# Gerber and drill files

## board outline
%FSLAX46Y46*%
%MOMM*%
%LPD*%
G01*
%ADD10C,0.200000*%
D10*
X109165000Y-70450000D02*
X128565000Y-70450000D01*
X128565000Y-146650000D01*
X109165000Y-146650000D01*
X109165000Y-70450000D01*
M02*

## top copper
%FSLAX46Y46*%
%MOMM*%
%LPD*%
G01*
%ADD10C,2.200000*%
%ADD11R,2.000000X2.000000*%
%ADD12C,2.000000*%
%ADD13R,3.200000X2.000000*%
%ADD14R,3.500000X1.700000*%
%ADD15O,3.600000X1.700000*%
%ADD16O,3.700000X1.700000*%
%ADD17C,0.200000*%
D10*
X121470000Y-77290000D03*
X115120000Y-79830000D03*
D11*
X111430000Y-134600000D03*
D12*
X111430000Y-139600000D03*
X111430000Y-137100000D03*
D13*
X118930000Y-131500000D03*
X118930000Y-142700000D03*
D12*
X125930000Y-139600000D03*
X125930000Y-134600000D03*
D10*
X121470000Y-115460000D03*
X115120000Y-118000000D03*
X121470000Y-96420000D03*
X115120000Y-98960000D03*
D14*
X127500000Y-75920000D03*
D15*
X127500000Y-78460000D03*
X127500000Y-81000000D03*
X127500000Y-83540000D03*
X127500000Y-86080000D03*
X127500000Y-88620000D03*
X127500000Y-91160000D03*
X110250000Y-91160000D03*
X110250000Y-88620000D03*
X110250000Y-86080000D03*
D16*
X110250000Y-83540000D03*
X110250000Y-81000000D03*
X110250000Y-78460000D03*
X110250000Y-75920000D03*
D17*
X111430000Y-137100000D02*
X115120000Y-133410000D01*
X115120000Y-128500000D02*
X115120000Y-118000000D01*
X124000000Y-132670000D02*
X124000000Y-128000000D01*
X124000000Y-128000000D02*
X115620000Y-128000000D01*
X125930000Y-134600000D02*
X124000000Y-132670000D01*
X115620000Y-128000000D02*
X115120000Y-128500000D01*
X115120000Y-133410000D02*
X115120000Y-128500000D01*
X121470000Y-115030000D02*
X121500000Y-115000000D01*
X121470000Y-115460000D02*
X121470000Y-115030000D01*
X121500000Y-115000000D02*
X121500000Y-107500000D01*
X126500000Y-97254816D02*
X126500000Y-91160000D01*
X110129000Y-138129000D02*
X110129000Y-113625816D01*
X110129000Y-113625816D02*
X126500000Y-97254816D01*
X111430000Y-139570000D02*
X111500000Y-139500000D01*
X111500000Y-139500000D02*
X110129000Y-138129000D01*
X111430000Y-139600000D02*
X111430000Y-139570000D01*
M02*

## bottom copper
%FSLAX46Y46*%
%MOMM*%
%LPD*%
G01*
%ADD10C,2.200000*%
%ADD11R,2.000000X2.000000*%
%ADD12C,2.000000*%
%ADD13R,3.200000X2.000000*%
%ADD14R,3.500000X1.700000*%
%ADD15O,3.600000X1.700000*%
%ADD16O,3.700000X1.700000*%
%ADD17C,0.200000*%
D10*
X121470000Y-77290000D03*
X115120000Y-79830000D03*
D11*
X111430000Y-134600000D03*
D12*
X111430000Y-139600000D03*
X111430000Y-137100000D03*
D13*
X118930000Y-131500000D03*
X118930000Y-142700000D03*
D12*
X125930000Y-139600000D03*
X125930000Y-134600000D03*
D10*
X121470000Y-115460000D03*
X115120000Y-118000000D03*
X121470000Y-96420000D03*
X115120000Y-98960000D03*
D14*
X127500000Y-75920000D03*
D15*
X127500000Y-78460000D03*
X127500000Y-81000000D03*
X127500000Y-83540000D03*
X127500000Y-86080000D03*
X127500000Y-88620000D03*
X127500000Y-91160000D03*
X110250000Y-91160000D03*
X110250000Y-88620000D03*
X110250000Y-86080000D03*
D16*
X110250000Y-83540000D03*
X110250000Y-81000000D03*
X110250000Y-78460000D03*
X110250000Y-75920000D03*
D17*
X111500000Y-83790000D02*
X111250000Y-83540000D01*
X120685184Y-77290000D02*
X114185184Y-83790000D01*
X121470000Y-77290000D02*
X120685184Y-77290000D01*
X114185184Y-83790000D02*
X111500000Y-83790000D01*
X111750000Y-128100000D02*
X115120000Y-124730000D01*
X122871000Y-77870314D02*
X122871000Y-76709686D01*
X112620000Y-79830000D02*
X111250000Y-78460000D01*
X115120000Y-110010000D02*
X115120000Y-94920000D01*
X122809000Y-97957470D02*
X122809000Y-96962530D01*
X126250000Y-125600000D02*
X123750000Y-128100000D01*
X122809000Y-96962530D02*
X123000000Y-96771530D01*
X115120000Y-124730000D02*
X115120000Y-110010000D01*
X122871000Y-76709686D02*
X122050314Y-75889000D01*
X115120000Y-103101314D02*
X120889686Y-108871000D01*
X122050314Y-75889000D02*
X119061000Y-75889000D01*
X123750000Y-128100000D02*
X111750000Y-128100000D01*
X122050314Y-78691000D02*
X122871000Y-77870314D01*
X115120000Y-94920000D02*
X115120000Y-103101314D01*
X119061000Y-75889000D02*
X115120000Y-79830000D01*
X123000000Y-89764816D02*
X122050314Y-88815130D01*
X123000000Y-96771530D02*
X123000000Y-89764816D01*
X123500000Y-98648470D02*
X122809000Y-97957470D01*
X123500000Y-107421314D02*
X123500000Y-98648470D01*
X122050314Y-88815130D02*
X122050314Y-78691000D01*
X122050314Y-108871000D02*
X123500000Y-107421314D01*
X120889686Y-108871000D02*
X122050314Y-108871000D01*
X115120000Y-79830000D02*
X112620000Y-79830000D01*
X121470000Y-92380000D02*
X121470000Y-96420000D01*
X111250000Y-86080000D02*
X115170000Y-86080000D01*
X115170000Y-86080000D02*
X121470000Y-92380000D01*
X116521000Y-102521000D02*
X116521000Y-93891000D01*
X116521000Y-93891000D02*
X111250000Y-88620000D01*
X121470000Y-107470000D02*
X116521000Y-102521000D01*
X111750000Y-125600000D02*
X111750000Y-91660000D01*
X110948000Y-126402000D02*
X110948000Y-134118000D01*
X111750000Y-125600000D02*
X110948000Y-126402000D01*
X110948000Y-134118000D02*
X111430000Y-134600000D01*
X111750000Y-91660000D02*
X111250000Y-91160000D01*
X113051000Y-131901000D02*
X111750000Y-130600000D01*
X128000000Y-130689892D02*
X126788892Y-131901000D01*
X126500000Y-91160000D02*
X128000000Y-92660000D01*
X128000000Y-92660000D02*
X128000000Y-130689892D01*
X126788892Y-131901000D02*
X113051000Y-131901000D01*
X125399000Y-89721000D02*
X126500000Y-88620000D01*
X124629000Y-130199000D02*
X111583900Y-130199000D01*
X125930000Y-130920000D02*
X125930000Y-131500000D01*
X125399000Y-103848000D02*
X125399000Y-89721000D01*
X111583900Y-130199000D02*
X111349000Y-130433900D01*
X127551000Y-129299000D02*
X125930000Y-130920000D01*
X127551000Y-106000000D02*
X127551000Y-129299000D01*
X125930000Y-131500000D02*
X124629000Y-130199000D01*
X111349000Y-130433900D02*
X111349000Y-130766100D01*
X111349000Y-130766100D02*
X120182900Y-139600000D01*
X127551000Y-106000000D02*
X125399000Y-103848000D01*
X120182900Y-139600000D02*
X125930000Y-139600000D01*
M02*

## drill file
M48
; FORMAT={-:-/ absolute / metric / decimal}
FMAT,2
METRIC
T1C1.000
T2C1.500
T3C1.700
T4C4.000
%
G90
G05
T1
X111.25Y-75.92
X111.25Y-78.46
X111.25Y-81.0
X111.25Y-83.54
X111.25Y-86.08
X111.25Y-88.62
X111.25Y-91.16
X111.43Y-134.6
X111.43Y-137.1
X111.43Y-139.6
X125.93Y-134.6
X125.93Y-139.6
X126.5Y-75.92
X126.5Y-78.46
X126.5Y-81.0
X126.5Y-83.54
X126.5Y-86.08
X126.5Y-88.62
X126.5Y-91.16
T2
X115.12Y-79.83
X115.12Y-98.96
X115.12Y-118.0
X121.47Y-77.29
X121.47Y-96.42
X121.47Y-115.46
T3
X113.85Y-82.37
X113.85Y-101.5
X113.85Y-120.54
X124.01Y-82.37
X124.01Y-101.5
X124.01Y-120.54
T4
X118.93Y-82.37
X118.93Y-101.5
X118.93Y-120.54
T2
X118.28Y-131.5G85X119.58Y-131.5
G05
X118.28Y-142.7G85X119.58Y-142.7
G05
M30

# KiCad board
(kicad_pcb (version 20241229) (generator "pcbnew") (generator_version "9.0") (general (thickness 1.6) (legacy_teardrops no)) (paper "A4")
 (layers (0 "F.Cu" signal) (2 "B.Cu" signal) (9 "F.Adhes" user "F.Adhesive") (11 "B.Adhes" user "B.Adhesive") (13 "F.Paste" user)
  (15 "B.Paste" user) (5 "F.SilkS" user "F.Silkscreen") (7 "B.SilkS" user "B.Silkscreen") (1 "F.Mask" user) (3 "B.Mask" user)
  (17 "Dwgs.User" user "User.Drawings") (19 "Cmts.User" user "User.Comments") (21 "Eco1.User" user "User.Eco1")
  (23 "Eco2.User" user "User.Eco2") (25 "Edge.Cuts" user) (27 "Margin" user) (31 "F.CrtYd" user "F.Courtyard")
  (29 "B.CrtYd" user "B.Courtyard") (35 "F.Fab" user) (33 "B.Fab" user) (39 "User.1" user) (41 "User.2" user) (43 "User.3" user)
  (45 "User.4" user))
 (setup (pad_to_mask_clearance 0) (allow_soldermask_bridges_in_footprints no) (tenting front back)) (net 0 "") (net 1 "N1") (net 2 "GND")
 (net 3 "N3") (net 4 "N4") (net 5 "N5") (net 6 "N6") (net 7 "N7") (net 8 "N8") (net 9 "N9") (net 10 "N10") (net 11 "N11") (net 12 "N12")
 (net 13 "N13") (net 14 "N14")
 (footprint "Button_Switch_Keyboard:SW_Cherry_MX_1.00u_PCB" (layer "F.Cu") (at 121.47 77.29)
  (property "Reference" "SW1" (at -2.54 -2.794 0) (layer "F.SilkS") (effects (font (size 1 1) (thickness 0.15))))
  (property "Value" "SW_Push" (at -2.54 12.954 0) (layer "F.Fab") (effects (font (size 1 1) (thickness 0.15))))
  (pad "" np_thru_hole circle (at -7.62 5.08) (size 1.7 1.7) (drill 1.7) (layers "*.Cu" "*.Mask"))
  (pad "" np_thru_hole circle (at -2.54 5.08) (size 4 4) (drill 4) (layers "*.Cu" "*.Mask"))
  (pad "" np_thru_hole circle (at 2.54 5.08) (size 1.7 1.7) (drill 1.7) (layers "*.Cu" "*.Mask"))
  (pad "1" thru_hole circle (at 0 0) (size 2.2 2.2) (drill 1.5) (layers "*.Cu" "*.Mask") (remove_unused_layers no) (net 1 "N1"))
  (pad "2" thru_hole circle (at -6.35 2.54) (size 2.2 2.2) (drill 1.5) (layers "*.Cu" "*.Mask") (remove_unused_layers no) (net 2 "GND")))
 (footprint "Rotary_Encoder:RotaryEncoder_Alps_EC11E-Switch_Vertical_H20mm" (layer "F.Cu") (at 111.43 134.6)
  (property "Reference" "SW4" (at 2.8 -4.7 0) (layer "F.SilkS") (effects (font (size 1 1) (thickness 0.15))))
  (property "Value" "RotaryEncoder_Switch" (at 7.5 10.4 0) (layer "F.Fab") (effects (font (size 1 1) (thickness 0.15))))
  (pad "A" thru_hole rect (at 0 0) (size 2 2) (drill 1) (layers "*.Cu" "*.Mask") (remove_unused_layers no) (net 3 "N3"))
  (pad "B" thru_hole circle (at 0 5) (size 2 2) (drill 1) (layers "*.Cu" "*.Mask") (remove_unused_layers no) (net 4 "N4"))
  (pad "C" thru_hole circle (at 0 2.5) (size 2 2) (drill 1) (layers "*.Cu" "*.Mask") (remove_unused_layers no) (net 2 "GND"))
  (pad "MP" thru_hole rect (at 7.5 -3.1) (size 3.2 2) (drill oval 2.8 1.5) (layers "*.Cu" "*.Mask") (remove_unused_layers no))
  (pad "MP" thru_hole rect (at 7.5 8.1) (size 3.2 2) (drill oval 2.8 1.5) (layers "*.Cu" "*.Mask") (remove_unused_layers no))
  (pad "S1" thru_hole circle (at 14.5 5) (size 2 2) (drill 1) (layers "*.Cu" "*.Mask") (remove_unused_layers no) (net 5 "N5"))
  (pad "S2" thru_hole circle (at 14.5 0) (size 2 2) (drill 1) (layers "*.Cu" "*.Mask") (remove_unused_layers no) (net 2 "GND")))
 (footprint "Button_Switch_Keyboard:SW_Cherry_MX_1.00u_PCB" (layer "F.Cu") (at 121.47 115.46)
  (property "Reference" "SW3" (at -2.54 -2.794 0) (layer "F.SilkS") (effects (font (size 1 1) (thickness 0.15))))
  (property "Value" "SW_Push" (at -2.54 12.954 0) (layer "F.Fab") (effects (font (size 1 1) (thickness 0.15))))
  (pad "" np_thru_hole circle (at -7.62 5.08) (size 1.7 1.7) (drill 1.7) (layers "*.Cu" "*.Mask"))
  (pad "" np_thru_hole circle (at -2.54 5.08) (size 4 4) (drill 4) (layers "*.Cu" "*.Mask"))
  (pad "" np_thru_hole circle (at 2.54 5.08) (size 1.7 1.7) (drill 1.7) (layers "*.Cu" "*.Mask"))
  (pad "1" thru_hole circle (at 0 0) (size 2.2 2.2) (drill 1.5) (layers "*.Cu" "*.Mask") (remove_unused_layers no) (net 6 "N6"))
  (pad "2" thru_hole circle (at -6.35 2.54) (size 2.2 2.2) (drill 1.5) (layers "*.Cu" "*.Mask") (remove_unused_layers no) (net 2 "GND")))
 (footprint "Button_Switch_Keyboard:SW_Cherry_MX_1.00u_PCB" (layer "F.Cu") (at 121.47 96.42)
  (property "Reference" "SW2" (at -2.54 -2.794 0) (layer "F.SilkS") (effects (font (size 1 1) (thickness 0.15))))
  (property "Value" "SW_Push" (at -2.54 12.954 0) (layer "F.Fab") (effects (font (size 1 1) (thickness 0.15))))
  (pad "" np_thru_hole circle (at -7.62 5.08) (size 1.7 1.7) (drill 1.7) (layers "*.Cu" "*.Mask"))
  (pad "" np_thru_hole circle (at -2.54 5.08) (size 4 4) (drill 4) (layers "*.Cu" "*.Mask"))
  (pad "" np_thru_hole circle (at 2.54 5.08) (size 1.7 1.7) (drill 1.7) (layers "*.Cu" "*.Mask"))
  (pad "1" thru_hole circle (at 0 0) (size 2.2 2.2) (drill 1.5) (layers "*.Cu" "*.Mask") (remove_unused_layers no) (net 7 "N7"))
  (pad "2" thru_hole circle (at -6.35 2.54) (size 2.2 2.2) (drill 1.5) (layers "*.Cu" "*.Mask") (remove_unused_layers no) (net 2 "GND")))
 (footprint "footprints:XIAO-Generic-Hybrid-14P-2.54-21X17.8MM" (layer "B.Cu") (at 118.875 83.54 180)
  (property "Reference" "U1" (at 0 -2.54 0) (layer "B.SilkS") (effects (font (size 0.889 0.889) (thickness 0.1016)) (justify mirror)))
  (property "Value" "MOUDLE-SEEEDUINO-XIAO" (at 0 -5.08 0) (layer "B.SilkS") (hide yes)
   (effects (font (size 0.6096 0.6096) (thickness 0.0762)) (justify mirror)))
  (pad "1" thru_hole rect (at -7.625 7.62 180) (size 3.5 1.7) (drill 1 (offset -1 0)) (layers "*.Cu" "*.Mask") (remove_unused_layers no)
   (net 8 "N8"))
  (pad "2" thru_hole oval (at -7.625 5.08 180) (size 3.6 1.7) (drill 1 (offset -1 0)) (layers "*.Cu" "*.Mask") (remove_unused_layers no)
   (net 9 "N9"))
  (pad "3" thru_hole oval (at -7.625 2.54 180) (size 3.6 1.7) (drill 1 (offset -1 0)) (layers "*.Cu" "*.Mask") (remove_unused_layers no)
   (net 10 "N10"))
  (pad "4" thru_hole oval (at -7.625 0 180) (size 3.6 1.7) (drill 1 (offset -1 0)) (layers "*.Cu" "*.Mask") (remove_unused_layers no)
   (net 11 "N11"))
  (pad "5" thru_hole oval (at -7.625 -2.54 180) (size 3.6 1.7) (drill 1 (offset -1 0)) (layers "*.Cu" "*.Mask") (remove_unused_layers no)
   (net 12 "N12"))
  (pad "6" thru_hole oval (at -7.625 -5.08) (size 3.6 1.7) (drill 1 (offset 1 0)) (layers "*.Cu" "*.Mask") (remove_unused_layers no)
   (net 5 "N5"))
  (pad "7" thru_hole oval (at -7.625 -7.62 180) (size 3.6 1.7) (drill 1 (offset -1 0)) (layers "*.Cu" "*.Mask") (remove_unused_layers no)
   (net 4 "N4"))
  (pad "8" thru_hole oval (at 7.625 -7.62 180) (size 3.6 1.7) (drill 1 (offset 1 0)) (layers "*.Cu" "*.Mask") (remove_unused_layers no)
   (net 3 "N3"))
  (pad "9" thru_hole oval (at 7.625 -5.08 180) (size 3.6 1.7) (drill 1 (offset 1 0)) (layers "*.Cu" "*.Mask") (remove_unused_layers no)
   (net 6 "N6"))
  (pad "10" thru_hole oval (at 7.625 -2.54 180) (size 3.6 1.7) (drill 1 (offset 1 0)) (layers "*.Cu" "*.Mask") (remove_unused_layers no)
   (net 7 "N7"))
  (pad "11" thru_hole oval (at 7.625 0 180) (size 3.7 1.7) (drill 1 (offset 1 0)) (layers "*.Cu" "*.Mask") (remove_unused_layers no)
   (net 1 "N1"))
  (pad "12" thru_hole oval (at 7.625 2.54 180) (size 3.7 1.7) (drill 1 (offset 1 0)) (layers "*.Cu" "*.Mask") (remove_unused_layers no)
   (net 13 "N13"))
  (pad "13" thru_hole oval (at 7.625 5.08 180) (size 3.7 1.7) (drill 1 (offset 1 0)) (layers "*.Cu" "*.Mask") (remove_unused_layers no)
   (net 2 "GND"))
  (pad "14" thru_hole oval (at 7.625 7.62 180) (size 3.7 1.7) (drill 1 (offset 1 0)) (layers "*.Cu" "*.Mask") (remove_unused_layers no)
   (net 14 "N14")))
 (gr_rect (start 109.165 70.45) (end 128.565 146.65) (stroke (width 0.2) (type solid)) (fill no) (layer "Edge.Cuts"))
 (segment (start 111.5 83.79) (end 111.25 83.54) (width 0.2) (layer "B.Cu") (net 1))
 (segment (start 120.685184 77.29) (end 114.185184 83.79) (width 0.2) (layer "B.Cu") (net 1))
 (segment (start 121.47 77.29) (end 120.685184 77.29) (width 0.2) (layer "B.Cu") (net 1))
 (segment (start 114.185184 83.79) (end 111.5 83.79) (width 0.2) (layer "B.Cu") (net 1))
 (segment (start 111.43 137.1) (end 115.12 133.41) (width 0.2) (layer "F.Cu") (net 2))
 (segment (start 115.12 128.5) (end 115.12 118) (width 0.2) (layer "F.Cu") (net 2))
 (segment (start 124 132.67) (end 124 128) (width 0.2) (layer "F.Cu") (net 2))
 (segment (start 124 128) (end 115.62 128) (width 0.2) (layer "F.Cu") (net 2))
 (segment (start 125.93 134.6) (end 124 132.67) (width 0.2) (layer "F.Cu") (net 2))
 (segment (start 115.62 128) (end 115.12 128.5) (width 0.2) (layer "F.Cu") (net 2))
 (segment (start 115.12 133.41) (end 115.12 128.5) (width 0.2) (layer "F.Cu") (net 2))
 (segment (start 111.75 128.1) (end 115.12 124.73) (width 0.2) (layer "B.Cu") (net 2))
 (segment (start 122.871 77.870314) (end 122.871 76.709686) (width 0.2) (layer "B.Cu") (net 2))
 (segment (start 112.62 79.83) (end 111.25 78.46) (width 0.2) (layer "B.Cu") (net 2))
 (segment (start 115.12 110.01) (end 115.12 94.92) (width 0.2) (layer "B.Cu") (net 2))
 (segment (start 122.809 97.95747) (end 122.809 96.96253) (width 0.2) (layer "B.Cu") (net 2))
 (segment (start 126.25 125.6) (end 123.75 128.1) (width 0.2) (layer "B.Cu") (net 2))
 (segment (start 122.809 96.96253) (end 123 96.77153) (width 0.2) (layer "B.Cu") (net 2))
 (segment (start 115.12 124.73) (end 115.12 110.01) (width 0.2) (layer "B.Cu") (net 2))
 (segment (start 122.871 76.709686) (end 122.050314 75.889) (width 0.2) (layer "B.Cu") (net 2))
 (segment (start 115.12 103.101314) (end 120.889686 108.871) (width 0.2) (layer "B.Cu") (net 2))
 (segment (start 122.050314 75.889) (end 119.061 75.889) (width 0.2) (layer "B.Cu") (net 2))
 (segment (start 123.75 128.1) (end 111.75 128.1) (width 0.2) (layer "B.Cu") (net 2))
 (segment (start 122.050314 78.691) (end 122.871 77.870314) (width 0.2) (layer "B.Cu") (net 2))
 (segment (start 115.12 94.92) (end 115.12 103.101314) (width 0.2) (layer "B.Cu") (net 2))
 (segment (start 119.061 75.889) (end 115.12 79.83) (width 0.2) (layer "B.Cu") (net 2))
 (segment (start 123 89.764816) (end 122.050314 88.81513) (width 0.2) (layer "B.Cu") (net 2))
 (segment (start 123 96.77153) (end 123 89.764816) (width 0.2) (layer "B.Cu") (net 2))
 (segment (start 123.5 98.64847) (end 122.809 97.95747) (width 0.2) (layer "B.Cu") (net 2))
 (segment (start 123.5 107.421314) (end 123.5 98.64847) (width 0.2) (layer "B.Cu") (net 2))
 (segment (start 122.050314 88.81513) (end 122.050314 78.691) (width 0.2) (layer "B.Cu") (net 2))
 (segment (start 122.050314 108.871) (end 123.5 107.421314) (width 0.2) (layer "B.Cu") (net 2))
 (segment (start 120.889686 108.871) (end 122.050314 108.871) (width 0.2) (layer "B.Cu") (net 2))
 (segment (start 115.12 79.83) (end 112.62 79.83) (width 0.2) (layer "B.Cu") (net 2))
 (segment (start 121.47 92.38) (end 121.47 96.42) (width 0.2) (layer "B.Cu") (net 7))
 (segment (start 111.25 86.08) (end 115.17 86.08) (width 0.2) (layer "B.Cu") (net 7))
 (segment (start 115.17 86.08) (end 121.47 92.38) (width 0.2) (layer "B.Cu") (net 7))
 (segment (start 121.47 115.03) (end 121.5 115) (width 0.2) (layer "F.Cu") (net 6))
 (segment (start 121.47 115.46) (end 121.47 115.03) (width 0.2) (layer "F.Cu") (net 6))
 (segment (start 121.5 115) (end 121.5 107.5) (width 0.2) (layer "F.Cu") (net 6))
 (segment (start 116.521 102.521) (end 116.521 93.891) (width 0.2) (layer "B.Cu") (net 6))
 (segment (start 116.521 93.891) (end 111.25 88.62) (width 0.2) (layer "B.Cu") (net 6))
 (segment (start 121.47 107.47) (end 116.521 102.521) (width 0.2) (layer "B.Cu") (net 6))
 (segment (start 111.75 125.6) (end 111.75 91.66) (width 0.2) (layer "B.Cu") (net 3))
 (segment (start 110.948 126.402) (end 110.948 134.118) (width 0.2) (layer "B.Cu") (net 3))
 (segment (start 111.75 125.6) (end 110.948 126.402) (width 0.2) (layer "B.Cu") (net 3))
 (segment (start 110.948 134.118) (end 111.43 134.6) (width 0.2) (layer "B.Cu") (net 3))
 (segment (start 111.75 91.66) (end 111.25 91.16) (width 0.2) (layer "B.Cu") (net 3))
 (segment (start 126.5 97.254816) (end 126.5 91.16) (width 0.2) (layer "F.Cu") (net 4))
 (segment (start 110.129 138.129) (end 110.129 113.625816) (width 0.2) (layer "F.Cu") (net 4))
 (segment (start 110.129 113.625816) (end 126.5 97.254816) (width 0.2) (layer "F.Cu") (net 4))
 (segment (start 111.43 139.57) (end 111.5 139.5) (width 0.2) (layer "F.Cu") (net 4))
 (segment (start 111.5 139.5) (end 110.129 138.129) (width 0.2) (layer "F.Cu") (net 4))
 (segment (start 111.43 139.6) (end 111.43 139.57) (width 0.2) (layer "F.Cu") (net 4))
 (segment (start 113.051 131.901) (end 111.75 130.6) (width 0.2) (layer "B.Cu") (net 4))
 (segment (start 128 130.689892) (end 126.788892 131.901) (width 0.2) (layer "B.Cu") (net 4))
 (segment (start 126.5 91.16) (end 128 92.66) (width 0.2) (layer "B.Cu") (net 4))
 (segment (start 128 92.66) (end 128 130.689892) (width 0.2) (layer "B.Cu") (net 4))
 (segment (start 126.788892 131.901) (end 113.051 131.901) (width 0.2) (layer "B.Cu") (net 4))
 (segment (start 125.399 89.721) (end 126.5 88.62) (width 0.2) (layer "B.Cu") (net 5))
 (segment (start 124.629 130.199) (end 111.5839 130.199) (width 0.2) (layer "B.Cu") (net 5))
 (segment (start 125.93 130.92) (end 125.93 131.5) (width 0.2) (layer "B.Cu") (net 5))
 (segment (start 125.399 103.848) (end 125.399 89.721) (width 0.2) (layer "B.Cu") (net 5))
 (segment (start 111.5839 130.199) (end 111.349 130.4339) (width 0.2) (layer "B.Cu") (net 5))
 (segment (start 127.551 129.299) (end 125.93 130.92) (width 0.2) (layer "B.Cu") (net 5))
 (segment (start 127.551 106) (end 127.551 129.299) (width 0.2) (layer "B.Cu") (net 5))
 (segment (start 125.93 131.5) (end 124.629 130.199) (width 0.2) (layer "B.Cu") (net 5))
 (segment (start 111.349 130.4339) (end 111.349 130.7661) (width 0.2) (layer "B.Cu") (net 5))
 (segment (start 111.349 130.7661) (end 120.1829 139.6) (width 0.2) (layer "B.Cu") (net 5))
 (segment (start 127.551 106) (end 125.399 103.848) (width 0.2) (layer "B.Cu") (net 5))
 (segment (start 120.1829 139.6) (end 125.93 139.6) (width 0.2) (layer "B.Cu") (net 5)))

